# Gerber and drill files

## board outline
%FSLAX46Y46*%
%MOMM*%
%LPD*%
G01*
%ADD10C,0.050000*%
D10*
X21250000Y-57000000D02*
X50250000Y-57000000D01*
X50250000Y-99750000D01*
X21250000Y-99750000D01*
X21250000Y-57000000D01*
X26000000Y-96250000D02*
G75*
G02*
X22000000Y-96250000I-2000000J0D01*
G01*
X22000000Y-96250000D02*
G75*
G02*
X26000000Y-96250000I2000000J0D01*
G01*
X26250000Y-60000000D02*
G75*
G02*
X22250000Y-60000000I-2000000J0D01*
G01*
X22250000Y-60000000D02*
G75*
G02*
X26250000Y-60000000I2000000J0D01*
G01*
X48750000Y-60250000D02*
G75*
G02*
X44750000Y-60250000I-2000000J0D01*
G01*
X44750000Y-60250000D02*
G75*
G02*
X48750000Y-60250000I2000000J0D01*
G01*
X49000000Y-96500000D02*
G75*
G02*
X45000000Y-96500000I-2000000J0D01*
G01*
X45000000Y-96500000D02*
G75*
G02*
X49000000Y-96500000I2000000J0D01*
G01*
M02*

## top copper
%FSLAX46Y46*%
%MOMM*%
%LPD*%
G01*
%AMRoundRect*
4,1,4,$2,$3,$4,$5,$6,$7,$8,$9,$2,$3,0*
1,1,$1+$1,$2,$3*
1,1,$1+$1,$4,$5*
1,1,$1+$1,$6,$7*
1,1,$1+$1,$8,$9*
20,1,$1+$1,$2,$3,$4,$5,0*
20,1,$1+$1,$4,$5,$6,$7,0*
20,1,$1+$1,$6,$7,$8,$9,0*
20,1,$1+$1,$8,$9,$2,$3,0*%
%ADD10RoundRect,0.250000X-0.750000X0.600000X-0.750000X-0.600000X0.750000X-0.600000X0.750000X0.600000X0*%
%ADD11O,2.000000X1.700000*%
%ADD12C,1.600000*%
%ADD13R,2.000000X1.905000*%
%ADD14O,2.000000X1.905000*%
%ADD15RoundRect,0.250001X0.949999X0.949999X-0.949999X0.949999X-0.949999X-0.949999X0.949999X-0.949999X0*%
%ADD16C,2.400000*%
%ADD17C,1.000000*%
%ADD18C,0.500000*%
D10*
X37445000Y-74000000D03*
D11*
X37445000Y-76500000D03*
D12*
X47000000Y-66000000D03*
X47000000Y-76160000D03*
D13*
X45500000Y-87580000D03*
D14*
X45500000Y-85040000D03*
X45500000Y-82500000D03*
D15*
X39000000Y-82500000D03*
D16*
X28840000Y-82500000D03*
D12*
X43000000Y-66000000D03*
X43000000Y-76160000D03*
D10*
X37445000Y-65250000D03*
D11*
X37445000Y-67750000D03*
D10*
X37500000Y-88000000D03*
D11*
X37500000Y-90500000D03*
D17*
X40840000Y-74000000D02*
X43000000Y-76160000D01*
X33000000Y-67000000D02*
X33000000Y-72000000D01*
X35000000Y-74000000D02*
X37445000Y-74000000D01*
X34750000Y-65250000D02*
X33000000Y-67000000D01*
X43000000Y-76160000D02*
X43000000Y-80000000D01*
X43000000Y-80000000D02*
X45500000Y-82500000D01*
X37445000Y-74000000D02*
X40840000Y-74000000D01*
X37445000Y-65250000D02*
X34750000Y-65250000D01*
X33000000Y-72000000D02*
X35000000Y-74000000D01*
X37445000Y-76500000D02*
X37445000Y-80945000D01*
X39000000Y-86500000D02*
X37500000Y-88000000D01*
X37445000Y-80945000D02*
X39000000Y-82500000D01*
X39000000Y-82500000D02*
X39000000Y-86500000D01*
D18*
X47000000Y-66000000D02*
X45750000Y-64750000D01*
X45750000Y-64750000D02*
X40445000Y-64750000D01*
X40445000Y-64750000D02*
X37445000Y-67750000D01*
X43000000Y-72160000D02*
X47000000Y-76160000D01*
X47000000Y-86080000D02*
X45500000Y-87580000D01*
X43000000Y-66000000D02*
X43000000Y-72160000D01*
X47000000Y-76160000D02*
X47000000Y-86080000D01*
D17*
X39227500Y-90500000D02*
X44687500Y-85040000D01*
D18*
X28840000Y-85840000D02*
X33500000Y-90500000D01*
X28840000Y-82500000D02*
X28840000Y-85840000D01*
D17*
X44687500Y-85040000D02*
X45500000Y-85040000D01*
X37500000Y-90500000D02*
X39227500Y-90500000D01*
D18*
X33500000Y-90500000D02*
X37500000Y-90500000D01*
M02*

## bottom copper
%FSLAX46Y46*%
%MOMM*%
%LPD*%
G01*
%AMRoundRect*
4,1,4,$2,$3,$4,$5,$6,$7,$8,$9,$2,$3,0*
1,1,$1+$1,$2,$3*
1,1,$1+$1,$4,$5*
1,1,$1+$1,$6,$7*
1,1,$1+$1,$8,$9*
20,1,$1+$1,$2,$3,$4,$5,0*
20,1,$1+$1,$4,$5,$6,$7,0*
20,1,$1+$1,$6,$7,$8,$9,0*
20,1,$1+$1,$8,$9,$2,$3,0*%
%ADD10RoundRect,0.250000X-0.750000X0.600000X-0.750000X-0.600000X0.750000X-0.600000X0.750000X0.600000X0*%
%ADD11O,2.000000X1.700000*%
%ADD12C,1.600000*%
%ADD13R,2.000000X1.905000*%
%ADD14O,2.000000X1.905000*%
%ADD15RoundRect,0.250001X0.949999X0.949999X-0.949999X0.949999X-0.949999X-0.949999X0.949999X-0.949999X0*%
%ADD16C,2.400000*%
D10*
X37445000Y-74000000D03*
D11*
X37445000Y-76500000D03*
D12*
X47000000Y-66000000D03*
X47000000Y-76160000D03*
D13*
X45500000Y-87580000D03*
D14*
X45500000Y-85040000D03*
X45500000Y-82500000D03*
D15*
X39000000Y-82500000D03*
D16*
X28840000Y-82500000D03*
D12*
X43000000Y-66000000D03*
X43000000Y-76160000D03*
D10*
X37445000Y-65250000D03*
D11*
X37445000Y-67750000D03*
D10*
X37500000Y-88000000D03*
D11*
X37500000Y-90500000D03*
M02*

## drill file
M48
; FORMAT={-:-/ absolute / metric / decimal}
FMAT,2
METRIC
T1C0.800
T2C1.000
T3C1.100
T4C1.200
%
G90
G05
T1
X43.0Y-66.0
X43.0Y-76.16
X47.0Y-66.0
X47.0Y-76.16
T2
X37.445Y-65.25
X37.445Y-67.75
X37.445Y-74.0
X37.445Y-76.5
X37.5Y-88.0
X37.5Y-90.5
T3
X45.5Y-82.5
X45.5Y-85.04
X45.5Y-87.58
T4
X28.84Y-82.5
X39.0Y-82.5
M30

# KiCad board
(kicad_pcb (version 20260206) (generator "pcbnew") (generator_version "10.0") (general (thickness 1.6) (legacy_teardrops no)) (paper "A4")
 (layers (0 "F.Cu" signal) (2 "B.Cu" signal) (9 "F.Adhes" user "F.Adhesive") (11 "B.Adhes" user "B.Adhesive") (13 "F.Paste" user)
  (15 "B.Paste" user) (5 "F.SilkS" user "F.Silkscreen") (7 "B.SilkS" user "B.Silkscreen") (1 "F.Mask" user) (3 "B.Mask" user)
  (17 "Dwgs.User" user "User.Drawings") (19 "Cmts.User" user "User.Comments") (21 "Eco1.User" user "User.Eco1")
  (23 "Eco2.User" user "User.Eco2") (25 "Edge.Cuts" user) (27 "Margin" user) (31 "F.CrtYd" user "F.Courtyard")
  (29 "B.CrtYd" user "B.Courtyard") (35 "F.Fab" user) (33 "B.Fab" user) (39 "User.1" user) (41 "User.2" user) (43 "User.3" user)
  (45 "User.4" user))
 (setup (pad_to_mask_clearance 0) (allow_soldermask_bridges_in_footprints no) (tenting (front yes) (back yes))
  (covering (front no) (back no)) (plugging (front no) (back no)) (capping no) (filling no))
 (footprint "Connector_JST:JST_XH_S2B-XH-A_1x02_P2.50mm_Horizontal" (layer "F.Cu") (at 37.445 74 -90)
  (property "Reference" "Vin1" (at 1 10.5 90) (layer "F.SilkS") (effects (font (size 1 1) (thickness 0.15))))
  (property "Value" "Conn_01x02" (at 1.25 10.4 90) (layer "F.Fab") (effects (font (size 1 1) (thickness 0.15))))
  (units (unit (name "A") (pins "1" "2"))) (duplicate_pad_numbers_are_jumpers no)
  (pad "1" thru_hole roundrect (at 0 0 270) (size 1.7 2) (drill 1) (layers "*.Cu" "*.Mask") (remove_unused_layers no)
   (roundrect_rratio 0.147059) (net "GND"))
  (pad "2" thru_hole oval (at 2.5 0 270) (size 1.7 2) (drill 1) (layers "*.Cu" "*.Mask") (remove_unused_layers no) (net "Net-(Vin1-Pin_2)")))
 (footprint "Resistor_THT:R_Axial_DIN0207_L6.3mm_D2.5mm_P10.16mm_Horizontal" (layer "F.Cu") (at 47 66 -90)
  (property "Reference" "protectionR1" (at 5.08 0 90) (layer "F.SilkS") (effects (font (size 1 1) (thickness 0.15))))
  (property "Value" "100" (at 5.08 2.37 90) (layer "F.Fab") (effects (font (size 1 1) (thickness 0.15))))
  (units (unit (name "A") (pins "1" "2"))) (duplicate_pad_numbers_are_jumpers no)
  (pad "1" thru_hole circle (at 0 0 270) (size 1.6 1.6) (drill 0.8) (layers "*.Cu" "*.Mask") (remove_unused_layers no)
   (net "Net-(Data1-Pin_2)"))
  (pad "2" thru_hole circle (at 10.16 0 270) (size 1.6 1.6) (drill 0.8) (layers "*.Cu" "*.Mask") (remove_unused_layers no)
   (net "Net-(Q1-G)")))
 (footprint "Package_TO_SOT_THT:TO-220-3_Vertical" (layer "F.Cu") (at 45.5 87.58 90)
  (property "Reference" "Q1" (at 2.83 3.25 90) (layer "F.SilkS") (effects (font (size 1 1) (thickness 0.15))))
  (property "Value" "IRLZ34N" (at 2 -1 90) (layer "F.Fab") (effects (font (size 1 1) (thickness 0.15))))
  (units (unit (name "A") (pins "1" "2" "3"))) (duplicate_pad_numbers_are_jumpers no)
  (pad "1" thru_hole rect (at 0 0 90) (size 1.905 2) (drill 1.1) (layers "*.Cu" "*.Mask") (remove_unused_layers no) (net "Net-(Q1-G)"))
  (pad "2" thru_hole oval (at 2.54 0 90) (size 1.905 2) (drill 1.1) (layers "*.Cu" "*.Mask") (remove_unused_layers no) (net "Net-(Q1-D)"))
  (pad "3" thru_hole oval (at 5.08 0 90) (size 1.905 2) (drill 1.1) (layers "*.Cu" "*.Mask") (remove_unused_layers no) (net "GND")))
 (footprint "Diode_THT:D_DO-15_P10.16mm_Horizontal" (layer "F.Cu") (at 39 82.5 180)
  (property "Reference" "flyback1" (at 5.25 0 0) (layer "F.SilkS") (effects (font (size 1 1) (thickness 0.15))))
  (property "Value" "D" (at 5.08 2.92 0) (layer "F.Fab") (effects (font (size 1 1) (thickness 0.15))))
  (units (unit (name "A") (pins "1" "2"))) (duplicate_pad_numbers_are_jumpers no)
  (pad "1" thru_hole roundrect (at 0 0 180) (size 2.4 2.4) (drill 1.2) (layers "*.Cu" "*.Mask") (remove_unused_layers no)
   (roundrect_rratio 0.104167) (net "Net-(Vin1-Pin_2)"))
  (pad "2" thru_hole circle (at 10.16 0 180) (size 2.4 2.4) (drill 1.2) (layers "*.Cu" "*.Mask") (remove_unused_layers no)
   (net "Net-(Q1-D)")))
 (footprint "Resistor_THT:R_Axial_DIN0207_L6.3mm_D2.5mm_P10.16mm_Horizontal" (layer "F.Cu") (at 43 66 -90)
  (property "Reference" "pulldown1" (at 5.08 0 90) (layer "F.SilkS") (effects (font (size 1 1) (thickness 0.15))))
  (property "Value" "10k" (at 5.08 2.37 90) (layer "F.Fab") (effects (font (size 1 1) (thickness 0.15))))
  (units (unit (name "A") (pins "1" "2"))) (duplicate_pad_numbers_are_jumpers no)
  (pad "1" thru_hole circle (at 0 0 270) (size 1.6 1.6) (drill 0.8) (layers "*.Cu" "*.Mask") (remove_unused_layers no) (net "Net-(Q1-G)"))
  (pad "2" thru_hole circle (at 10.16 0 270) (size 1.6 1.6) (drill 0.8) (layers "*.Cu" "*.Mask") (remove_unused_layers no) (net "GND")))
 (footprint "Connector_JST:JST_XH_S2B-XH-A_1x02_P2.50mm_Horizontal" (layer "F.Cu") (at 37.445 65.25 -90)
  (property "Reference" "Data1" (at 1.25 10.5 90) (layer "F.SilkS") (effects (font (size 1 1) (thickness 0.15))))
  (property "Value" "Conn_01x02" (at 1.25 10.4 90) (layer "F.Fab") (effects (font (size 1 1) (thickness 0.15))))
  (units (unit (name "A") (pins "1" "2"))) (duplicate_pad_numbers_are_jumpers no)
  (pad "1" thru_hole roundrect (at 0 0 270) (size 1.7 2) (drill 1) (layers "*.Cu" "*.Mask") (remove_unused_layers no)
   (roundrect_rratio 0.147059) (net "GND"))
  (pad "2" thru_hole oval (at 2.5 0 270) (size 1.7 2) (drill 1) (layers "*.Cu" "*.Mask") (remove_unused_layers no) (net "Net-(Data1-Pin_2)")))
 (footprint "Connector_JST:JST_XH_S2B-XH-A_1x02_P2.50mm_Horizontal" (layer "F.Cu") (at 37.5 88 -90)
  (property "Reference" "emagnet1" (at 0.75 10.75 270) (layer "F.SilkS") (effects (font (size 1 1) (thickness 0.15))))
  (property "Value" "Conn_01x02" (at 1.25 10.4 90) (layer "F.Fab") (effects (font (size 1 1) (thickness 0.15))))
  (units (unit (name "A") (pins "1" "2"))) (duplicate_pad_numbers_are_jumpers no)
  (pad "1" thru_hole roundrect (at 0 0 270) (size 1.7 2) (drill 1) (layers "*.Cu" "*.Mask") (remove_unused_layers no)
   (roundrect_rratio 0.147059) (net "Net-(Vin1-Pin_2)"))
  (pad "2" thru_hole oval (at 2.5 0 270) (size 1.7 2) (drill 1) (layers "*.Cu" "*.Mask") (remove_unused_layers no) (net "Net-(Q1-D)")))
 (gr_rect (start 21.25 57) (end 50.25 99.75) (stroke (width 0.05) (type default)) (fill no) (layer "Edge.Cuts"))
 (gr_circle (center 24 96.25) (end 26 96.25) (stroke (width 0.05) (type default)) (fill no) (layer "Edge.Cuts"))
 (gr_circle (center 24.25 60) (end 26.25 60) (stroke (width 0.05) (type solid)) (fill no) (layer "Edge.Cuts"))
 (gr_circle (center 46.75 60.25) (end 48.75 60.25) (stroke (width 0.05) (type default)) (fill no) (layer "Edge.Cuts"))
 (gr_circle (center 47 96.5) (end 47 94.5) (stroke (width 0.05) (type default)) (fill no) (layer "Edge.Cuts"))
 (segment (start 40.84 74) (end 43 76.16) (width 1) (layer "F.Cu") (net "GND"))
 (segment (start 33 67) (end 33 72) (width 1) (layer "F.Cu") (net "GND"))
 (segment (start 35 74) (end 37.445 74) (width 1) (layer "F.Cu") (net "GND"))
 (segment (start 34.75 65.25) (end 33 67) (width 1) (layer "F.Cu") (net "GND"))
 (segment (start 43 76.16) (end 43 80) (width 1) (layer "F.Cu") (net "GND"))
 (segment (start 43 80) (end 45.5 82.5) (width 1) (layer "F.Cu") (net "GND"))
 (segment (start 37.445 74) (end 40.84 74) (width 1) (layer "F.Cu") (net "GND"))
 (segment (start 37.445 65.25) (end 34.75 65.25) (width 1) (layer "F.Cu") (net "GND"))
 (segment (start 33 72) (end 35 74) (width 1) (layer "F.Cu") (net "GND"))
 (segment (start 37.445 76.5) (end 37.445 80.945) (width 1) (layer "F.Cu") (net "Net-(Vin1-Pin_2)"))
 (segment (start 39 86.5) (end 37.5 88) (width 1) (layer "F.Cu") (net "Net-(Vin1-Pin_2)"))
 (segment (start 37.445 80.945) (end 39 82.5) (width 1) (layer "F.Cu") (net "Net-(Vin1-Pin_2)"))
 (segment (start 39 82.5) (end 39 86.5) (width 1) (layer "F.Cu") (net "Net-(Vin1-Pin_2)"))
 (segment (start 47 66) (end 45.75 64.75) (width 0.5) (layer "F.Cu") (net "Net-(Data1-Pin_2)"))
 (segment (start 45.75 64.75) (end 40.445 64.75) (width 0.5) (layer "F.Cu") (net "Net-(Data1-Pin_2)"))
 (segment (start 40.445 64.75) (end 37.445 67.75) (width 0.5) (layer "F.Cu") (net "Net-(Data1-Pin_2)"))
 (segment (start 43 72.16) (end 47 76.16) (width 0.5) (layer "F.Cu") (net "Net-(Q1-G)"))
 (segment (start 47 86.08) (end 45.5 87.58) (width 0.5) (layer "F.Cu") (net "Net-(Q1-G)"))
 (segment (start 43 66) (end 43 72.16) (width 0.5) (layer "F.Cu") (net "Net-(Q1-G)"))
 (segment (start 47 76.16) (end 47 86.08) (width 0.5) (layer "F.Cu") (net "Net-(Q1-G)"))
 (segment (start 39.2275 90.5) (end 44.6875 85.04) (width 1) (layer "F.Cu") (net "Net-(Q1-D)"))
 (segment (start 28.84 85.84) (end 33.5 90.5) (width 0.5) (layer "F.Cu") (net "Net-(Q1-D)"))
 (segment (start 28.84 82.5) (end 28.84 85.84) (width 0.5) (layer "F.Cu") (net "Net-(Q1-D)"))
 (segment (start 44.6875 85.04) (end 45.5 85.04) (width 1) (layer "F.Cu") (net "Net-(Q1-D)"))
 (segment (start 37.5 90.5) (end 39.2275 90.5) (width 1) (layer "F.Cu") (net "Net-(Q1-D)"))
 (segment (start 33.5 90.5) (end 37.5 90.5) (width 0.5) (layer "F.Cu") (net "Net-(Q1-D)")))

